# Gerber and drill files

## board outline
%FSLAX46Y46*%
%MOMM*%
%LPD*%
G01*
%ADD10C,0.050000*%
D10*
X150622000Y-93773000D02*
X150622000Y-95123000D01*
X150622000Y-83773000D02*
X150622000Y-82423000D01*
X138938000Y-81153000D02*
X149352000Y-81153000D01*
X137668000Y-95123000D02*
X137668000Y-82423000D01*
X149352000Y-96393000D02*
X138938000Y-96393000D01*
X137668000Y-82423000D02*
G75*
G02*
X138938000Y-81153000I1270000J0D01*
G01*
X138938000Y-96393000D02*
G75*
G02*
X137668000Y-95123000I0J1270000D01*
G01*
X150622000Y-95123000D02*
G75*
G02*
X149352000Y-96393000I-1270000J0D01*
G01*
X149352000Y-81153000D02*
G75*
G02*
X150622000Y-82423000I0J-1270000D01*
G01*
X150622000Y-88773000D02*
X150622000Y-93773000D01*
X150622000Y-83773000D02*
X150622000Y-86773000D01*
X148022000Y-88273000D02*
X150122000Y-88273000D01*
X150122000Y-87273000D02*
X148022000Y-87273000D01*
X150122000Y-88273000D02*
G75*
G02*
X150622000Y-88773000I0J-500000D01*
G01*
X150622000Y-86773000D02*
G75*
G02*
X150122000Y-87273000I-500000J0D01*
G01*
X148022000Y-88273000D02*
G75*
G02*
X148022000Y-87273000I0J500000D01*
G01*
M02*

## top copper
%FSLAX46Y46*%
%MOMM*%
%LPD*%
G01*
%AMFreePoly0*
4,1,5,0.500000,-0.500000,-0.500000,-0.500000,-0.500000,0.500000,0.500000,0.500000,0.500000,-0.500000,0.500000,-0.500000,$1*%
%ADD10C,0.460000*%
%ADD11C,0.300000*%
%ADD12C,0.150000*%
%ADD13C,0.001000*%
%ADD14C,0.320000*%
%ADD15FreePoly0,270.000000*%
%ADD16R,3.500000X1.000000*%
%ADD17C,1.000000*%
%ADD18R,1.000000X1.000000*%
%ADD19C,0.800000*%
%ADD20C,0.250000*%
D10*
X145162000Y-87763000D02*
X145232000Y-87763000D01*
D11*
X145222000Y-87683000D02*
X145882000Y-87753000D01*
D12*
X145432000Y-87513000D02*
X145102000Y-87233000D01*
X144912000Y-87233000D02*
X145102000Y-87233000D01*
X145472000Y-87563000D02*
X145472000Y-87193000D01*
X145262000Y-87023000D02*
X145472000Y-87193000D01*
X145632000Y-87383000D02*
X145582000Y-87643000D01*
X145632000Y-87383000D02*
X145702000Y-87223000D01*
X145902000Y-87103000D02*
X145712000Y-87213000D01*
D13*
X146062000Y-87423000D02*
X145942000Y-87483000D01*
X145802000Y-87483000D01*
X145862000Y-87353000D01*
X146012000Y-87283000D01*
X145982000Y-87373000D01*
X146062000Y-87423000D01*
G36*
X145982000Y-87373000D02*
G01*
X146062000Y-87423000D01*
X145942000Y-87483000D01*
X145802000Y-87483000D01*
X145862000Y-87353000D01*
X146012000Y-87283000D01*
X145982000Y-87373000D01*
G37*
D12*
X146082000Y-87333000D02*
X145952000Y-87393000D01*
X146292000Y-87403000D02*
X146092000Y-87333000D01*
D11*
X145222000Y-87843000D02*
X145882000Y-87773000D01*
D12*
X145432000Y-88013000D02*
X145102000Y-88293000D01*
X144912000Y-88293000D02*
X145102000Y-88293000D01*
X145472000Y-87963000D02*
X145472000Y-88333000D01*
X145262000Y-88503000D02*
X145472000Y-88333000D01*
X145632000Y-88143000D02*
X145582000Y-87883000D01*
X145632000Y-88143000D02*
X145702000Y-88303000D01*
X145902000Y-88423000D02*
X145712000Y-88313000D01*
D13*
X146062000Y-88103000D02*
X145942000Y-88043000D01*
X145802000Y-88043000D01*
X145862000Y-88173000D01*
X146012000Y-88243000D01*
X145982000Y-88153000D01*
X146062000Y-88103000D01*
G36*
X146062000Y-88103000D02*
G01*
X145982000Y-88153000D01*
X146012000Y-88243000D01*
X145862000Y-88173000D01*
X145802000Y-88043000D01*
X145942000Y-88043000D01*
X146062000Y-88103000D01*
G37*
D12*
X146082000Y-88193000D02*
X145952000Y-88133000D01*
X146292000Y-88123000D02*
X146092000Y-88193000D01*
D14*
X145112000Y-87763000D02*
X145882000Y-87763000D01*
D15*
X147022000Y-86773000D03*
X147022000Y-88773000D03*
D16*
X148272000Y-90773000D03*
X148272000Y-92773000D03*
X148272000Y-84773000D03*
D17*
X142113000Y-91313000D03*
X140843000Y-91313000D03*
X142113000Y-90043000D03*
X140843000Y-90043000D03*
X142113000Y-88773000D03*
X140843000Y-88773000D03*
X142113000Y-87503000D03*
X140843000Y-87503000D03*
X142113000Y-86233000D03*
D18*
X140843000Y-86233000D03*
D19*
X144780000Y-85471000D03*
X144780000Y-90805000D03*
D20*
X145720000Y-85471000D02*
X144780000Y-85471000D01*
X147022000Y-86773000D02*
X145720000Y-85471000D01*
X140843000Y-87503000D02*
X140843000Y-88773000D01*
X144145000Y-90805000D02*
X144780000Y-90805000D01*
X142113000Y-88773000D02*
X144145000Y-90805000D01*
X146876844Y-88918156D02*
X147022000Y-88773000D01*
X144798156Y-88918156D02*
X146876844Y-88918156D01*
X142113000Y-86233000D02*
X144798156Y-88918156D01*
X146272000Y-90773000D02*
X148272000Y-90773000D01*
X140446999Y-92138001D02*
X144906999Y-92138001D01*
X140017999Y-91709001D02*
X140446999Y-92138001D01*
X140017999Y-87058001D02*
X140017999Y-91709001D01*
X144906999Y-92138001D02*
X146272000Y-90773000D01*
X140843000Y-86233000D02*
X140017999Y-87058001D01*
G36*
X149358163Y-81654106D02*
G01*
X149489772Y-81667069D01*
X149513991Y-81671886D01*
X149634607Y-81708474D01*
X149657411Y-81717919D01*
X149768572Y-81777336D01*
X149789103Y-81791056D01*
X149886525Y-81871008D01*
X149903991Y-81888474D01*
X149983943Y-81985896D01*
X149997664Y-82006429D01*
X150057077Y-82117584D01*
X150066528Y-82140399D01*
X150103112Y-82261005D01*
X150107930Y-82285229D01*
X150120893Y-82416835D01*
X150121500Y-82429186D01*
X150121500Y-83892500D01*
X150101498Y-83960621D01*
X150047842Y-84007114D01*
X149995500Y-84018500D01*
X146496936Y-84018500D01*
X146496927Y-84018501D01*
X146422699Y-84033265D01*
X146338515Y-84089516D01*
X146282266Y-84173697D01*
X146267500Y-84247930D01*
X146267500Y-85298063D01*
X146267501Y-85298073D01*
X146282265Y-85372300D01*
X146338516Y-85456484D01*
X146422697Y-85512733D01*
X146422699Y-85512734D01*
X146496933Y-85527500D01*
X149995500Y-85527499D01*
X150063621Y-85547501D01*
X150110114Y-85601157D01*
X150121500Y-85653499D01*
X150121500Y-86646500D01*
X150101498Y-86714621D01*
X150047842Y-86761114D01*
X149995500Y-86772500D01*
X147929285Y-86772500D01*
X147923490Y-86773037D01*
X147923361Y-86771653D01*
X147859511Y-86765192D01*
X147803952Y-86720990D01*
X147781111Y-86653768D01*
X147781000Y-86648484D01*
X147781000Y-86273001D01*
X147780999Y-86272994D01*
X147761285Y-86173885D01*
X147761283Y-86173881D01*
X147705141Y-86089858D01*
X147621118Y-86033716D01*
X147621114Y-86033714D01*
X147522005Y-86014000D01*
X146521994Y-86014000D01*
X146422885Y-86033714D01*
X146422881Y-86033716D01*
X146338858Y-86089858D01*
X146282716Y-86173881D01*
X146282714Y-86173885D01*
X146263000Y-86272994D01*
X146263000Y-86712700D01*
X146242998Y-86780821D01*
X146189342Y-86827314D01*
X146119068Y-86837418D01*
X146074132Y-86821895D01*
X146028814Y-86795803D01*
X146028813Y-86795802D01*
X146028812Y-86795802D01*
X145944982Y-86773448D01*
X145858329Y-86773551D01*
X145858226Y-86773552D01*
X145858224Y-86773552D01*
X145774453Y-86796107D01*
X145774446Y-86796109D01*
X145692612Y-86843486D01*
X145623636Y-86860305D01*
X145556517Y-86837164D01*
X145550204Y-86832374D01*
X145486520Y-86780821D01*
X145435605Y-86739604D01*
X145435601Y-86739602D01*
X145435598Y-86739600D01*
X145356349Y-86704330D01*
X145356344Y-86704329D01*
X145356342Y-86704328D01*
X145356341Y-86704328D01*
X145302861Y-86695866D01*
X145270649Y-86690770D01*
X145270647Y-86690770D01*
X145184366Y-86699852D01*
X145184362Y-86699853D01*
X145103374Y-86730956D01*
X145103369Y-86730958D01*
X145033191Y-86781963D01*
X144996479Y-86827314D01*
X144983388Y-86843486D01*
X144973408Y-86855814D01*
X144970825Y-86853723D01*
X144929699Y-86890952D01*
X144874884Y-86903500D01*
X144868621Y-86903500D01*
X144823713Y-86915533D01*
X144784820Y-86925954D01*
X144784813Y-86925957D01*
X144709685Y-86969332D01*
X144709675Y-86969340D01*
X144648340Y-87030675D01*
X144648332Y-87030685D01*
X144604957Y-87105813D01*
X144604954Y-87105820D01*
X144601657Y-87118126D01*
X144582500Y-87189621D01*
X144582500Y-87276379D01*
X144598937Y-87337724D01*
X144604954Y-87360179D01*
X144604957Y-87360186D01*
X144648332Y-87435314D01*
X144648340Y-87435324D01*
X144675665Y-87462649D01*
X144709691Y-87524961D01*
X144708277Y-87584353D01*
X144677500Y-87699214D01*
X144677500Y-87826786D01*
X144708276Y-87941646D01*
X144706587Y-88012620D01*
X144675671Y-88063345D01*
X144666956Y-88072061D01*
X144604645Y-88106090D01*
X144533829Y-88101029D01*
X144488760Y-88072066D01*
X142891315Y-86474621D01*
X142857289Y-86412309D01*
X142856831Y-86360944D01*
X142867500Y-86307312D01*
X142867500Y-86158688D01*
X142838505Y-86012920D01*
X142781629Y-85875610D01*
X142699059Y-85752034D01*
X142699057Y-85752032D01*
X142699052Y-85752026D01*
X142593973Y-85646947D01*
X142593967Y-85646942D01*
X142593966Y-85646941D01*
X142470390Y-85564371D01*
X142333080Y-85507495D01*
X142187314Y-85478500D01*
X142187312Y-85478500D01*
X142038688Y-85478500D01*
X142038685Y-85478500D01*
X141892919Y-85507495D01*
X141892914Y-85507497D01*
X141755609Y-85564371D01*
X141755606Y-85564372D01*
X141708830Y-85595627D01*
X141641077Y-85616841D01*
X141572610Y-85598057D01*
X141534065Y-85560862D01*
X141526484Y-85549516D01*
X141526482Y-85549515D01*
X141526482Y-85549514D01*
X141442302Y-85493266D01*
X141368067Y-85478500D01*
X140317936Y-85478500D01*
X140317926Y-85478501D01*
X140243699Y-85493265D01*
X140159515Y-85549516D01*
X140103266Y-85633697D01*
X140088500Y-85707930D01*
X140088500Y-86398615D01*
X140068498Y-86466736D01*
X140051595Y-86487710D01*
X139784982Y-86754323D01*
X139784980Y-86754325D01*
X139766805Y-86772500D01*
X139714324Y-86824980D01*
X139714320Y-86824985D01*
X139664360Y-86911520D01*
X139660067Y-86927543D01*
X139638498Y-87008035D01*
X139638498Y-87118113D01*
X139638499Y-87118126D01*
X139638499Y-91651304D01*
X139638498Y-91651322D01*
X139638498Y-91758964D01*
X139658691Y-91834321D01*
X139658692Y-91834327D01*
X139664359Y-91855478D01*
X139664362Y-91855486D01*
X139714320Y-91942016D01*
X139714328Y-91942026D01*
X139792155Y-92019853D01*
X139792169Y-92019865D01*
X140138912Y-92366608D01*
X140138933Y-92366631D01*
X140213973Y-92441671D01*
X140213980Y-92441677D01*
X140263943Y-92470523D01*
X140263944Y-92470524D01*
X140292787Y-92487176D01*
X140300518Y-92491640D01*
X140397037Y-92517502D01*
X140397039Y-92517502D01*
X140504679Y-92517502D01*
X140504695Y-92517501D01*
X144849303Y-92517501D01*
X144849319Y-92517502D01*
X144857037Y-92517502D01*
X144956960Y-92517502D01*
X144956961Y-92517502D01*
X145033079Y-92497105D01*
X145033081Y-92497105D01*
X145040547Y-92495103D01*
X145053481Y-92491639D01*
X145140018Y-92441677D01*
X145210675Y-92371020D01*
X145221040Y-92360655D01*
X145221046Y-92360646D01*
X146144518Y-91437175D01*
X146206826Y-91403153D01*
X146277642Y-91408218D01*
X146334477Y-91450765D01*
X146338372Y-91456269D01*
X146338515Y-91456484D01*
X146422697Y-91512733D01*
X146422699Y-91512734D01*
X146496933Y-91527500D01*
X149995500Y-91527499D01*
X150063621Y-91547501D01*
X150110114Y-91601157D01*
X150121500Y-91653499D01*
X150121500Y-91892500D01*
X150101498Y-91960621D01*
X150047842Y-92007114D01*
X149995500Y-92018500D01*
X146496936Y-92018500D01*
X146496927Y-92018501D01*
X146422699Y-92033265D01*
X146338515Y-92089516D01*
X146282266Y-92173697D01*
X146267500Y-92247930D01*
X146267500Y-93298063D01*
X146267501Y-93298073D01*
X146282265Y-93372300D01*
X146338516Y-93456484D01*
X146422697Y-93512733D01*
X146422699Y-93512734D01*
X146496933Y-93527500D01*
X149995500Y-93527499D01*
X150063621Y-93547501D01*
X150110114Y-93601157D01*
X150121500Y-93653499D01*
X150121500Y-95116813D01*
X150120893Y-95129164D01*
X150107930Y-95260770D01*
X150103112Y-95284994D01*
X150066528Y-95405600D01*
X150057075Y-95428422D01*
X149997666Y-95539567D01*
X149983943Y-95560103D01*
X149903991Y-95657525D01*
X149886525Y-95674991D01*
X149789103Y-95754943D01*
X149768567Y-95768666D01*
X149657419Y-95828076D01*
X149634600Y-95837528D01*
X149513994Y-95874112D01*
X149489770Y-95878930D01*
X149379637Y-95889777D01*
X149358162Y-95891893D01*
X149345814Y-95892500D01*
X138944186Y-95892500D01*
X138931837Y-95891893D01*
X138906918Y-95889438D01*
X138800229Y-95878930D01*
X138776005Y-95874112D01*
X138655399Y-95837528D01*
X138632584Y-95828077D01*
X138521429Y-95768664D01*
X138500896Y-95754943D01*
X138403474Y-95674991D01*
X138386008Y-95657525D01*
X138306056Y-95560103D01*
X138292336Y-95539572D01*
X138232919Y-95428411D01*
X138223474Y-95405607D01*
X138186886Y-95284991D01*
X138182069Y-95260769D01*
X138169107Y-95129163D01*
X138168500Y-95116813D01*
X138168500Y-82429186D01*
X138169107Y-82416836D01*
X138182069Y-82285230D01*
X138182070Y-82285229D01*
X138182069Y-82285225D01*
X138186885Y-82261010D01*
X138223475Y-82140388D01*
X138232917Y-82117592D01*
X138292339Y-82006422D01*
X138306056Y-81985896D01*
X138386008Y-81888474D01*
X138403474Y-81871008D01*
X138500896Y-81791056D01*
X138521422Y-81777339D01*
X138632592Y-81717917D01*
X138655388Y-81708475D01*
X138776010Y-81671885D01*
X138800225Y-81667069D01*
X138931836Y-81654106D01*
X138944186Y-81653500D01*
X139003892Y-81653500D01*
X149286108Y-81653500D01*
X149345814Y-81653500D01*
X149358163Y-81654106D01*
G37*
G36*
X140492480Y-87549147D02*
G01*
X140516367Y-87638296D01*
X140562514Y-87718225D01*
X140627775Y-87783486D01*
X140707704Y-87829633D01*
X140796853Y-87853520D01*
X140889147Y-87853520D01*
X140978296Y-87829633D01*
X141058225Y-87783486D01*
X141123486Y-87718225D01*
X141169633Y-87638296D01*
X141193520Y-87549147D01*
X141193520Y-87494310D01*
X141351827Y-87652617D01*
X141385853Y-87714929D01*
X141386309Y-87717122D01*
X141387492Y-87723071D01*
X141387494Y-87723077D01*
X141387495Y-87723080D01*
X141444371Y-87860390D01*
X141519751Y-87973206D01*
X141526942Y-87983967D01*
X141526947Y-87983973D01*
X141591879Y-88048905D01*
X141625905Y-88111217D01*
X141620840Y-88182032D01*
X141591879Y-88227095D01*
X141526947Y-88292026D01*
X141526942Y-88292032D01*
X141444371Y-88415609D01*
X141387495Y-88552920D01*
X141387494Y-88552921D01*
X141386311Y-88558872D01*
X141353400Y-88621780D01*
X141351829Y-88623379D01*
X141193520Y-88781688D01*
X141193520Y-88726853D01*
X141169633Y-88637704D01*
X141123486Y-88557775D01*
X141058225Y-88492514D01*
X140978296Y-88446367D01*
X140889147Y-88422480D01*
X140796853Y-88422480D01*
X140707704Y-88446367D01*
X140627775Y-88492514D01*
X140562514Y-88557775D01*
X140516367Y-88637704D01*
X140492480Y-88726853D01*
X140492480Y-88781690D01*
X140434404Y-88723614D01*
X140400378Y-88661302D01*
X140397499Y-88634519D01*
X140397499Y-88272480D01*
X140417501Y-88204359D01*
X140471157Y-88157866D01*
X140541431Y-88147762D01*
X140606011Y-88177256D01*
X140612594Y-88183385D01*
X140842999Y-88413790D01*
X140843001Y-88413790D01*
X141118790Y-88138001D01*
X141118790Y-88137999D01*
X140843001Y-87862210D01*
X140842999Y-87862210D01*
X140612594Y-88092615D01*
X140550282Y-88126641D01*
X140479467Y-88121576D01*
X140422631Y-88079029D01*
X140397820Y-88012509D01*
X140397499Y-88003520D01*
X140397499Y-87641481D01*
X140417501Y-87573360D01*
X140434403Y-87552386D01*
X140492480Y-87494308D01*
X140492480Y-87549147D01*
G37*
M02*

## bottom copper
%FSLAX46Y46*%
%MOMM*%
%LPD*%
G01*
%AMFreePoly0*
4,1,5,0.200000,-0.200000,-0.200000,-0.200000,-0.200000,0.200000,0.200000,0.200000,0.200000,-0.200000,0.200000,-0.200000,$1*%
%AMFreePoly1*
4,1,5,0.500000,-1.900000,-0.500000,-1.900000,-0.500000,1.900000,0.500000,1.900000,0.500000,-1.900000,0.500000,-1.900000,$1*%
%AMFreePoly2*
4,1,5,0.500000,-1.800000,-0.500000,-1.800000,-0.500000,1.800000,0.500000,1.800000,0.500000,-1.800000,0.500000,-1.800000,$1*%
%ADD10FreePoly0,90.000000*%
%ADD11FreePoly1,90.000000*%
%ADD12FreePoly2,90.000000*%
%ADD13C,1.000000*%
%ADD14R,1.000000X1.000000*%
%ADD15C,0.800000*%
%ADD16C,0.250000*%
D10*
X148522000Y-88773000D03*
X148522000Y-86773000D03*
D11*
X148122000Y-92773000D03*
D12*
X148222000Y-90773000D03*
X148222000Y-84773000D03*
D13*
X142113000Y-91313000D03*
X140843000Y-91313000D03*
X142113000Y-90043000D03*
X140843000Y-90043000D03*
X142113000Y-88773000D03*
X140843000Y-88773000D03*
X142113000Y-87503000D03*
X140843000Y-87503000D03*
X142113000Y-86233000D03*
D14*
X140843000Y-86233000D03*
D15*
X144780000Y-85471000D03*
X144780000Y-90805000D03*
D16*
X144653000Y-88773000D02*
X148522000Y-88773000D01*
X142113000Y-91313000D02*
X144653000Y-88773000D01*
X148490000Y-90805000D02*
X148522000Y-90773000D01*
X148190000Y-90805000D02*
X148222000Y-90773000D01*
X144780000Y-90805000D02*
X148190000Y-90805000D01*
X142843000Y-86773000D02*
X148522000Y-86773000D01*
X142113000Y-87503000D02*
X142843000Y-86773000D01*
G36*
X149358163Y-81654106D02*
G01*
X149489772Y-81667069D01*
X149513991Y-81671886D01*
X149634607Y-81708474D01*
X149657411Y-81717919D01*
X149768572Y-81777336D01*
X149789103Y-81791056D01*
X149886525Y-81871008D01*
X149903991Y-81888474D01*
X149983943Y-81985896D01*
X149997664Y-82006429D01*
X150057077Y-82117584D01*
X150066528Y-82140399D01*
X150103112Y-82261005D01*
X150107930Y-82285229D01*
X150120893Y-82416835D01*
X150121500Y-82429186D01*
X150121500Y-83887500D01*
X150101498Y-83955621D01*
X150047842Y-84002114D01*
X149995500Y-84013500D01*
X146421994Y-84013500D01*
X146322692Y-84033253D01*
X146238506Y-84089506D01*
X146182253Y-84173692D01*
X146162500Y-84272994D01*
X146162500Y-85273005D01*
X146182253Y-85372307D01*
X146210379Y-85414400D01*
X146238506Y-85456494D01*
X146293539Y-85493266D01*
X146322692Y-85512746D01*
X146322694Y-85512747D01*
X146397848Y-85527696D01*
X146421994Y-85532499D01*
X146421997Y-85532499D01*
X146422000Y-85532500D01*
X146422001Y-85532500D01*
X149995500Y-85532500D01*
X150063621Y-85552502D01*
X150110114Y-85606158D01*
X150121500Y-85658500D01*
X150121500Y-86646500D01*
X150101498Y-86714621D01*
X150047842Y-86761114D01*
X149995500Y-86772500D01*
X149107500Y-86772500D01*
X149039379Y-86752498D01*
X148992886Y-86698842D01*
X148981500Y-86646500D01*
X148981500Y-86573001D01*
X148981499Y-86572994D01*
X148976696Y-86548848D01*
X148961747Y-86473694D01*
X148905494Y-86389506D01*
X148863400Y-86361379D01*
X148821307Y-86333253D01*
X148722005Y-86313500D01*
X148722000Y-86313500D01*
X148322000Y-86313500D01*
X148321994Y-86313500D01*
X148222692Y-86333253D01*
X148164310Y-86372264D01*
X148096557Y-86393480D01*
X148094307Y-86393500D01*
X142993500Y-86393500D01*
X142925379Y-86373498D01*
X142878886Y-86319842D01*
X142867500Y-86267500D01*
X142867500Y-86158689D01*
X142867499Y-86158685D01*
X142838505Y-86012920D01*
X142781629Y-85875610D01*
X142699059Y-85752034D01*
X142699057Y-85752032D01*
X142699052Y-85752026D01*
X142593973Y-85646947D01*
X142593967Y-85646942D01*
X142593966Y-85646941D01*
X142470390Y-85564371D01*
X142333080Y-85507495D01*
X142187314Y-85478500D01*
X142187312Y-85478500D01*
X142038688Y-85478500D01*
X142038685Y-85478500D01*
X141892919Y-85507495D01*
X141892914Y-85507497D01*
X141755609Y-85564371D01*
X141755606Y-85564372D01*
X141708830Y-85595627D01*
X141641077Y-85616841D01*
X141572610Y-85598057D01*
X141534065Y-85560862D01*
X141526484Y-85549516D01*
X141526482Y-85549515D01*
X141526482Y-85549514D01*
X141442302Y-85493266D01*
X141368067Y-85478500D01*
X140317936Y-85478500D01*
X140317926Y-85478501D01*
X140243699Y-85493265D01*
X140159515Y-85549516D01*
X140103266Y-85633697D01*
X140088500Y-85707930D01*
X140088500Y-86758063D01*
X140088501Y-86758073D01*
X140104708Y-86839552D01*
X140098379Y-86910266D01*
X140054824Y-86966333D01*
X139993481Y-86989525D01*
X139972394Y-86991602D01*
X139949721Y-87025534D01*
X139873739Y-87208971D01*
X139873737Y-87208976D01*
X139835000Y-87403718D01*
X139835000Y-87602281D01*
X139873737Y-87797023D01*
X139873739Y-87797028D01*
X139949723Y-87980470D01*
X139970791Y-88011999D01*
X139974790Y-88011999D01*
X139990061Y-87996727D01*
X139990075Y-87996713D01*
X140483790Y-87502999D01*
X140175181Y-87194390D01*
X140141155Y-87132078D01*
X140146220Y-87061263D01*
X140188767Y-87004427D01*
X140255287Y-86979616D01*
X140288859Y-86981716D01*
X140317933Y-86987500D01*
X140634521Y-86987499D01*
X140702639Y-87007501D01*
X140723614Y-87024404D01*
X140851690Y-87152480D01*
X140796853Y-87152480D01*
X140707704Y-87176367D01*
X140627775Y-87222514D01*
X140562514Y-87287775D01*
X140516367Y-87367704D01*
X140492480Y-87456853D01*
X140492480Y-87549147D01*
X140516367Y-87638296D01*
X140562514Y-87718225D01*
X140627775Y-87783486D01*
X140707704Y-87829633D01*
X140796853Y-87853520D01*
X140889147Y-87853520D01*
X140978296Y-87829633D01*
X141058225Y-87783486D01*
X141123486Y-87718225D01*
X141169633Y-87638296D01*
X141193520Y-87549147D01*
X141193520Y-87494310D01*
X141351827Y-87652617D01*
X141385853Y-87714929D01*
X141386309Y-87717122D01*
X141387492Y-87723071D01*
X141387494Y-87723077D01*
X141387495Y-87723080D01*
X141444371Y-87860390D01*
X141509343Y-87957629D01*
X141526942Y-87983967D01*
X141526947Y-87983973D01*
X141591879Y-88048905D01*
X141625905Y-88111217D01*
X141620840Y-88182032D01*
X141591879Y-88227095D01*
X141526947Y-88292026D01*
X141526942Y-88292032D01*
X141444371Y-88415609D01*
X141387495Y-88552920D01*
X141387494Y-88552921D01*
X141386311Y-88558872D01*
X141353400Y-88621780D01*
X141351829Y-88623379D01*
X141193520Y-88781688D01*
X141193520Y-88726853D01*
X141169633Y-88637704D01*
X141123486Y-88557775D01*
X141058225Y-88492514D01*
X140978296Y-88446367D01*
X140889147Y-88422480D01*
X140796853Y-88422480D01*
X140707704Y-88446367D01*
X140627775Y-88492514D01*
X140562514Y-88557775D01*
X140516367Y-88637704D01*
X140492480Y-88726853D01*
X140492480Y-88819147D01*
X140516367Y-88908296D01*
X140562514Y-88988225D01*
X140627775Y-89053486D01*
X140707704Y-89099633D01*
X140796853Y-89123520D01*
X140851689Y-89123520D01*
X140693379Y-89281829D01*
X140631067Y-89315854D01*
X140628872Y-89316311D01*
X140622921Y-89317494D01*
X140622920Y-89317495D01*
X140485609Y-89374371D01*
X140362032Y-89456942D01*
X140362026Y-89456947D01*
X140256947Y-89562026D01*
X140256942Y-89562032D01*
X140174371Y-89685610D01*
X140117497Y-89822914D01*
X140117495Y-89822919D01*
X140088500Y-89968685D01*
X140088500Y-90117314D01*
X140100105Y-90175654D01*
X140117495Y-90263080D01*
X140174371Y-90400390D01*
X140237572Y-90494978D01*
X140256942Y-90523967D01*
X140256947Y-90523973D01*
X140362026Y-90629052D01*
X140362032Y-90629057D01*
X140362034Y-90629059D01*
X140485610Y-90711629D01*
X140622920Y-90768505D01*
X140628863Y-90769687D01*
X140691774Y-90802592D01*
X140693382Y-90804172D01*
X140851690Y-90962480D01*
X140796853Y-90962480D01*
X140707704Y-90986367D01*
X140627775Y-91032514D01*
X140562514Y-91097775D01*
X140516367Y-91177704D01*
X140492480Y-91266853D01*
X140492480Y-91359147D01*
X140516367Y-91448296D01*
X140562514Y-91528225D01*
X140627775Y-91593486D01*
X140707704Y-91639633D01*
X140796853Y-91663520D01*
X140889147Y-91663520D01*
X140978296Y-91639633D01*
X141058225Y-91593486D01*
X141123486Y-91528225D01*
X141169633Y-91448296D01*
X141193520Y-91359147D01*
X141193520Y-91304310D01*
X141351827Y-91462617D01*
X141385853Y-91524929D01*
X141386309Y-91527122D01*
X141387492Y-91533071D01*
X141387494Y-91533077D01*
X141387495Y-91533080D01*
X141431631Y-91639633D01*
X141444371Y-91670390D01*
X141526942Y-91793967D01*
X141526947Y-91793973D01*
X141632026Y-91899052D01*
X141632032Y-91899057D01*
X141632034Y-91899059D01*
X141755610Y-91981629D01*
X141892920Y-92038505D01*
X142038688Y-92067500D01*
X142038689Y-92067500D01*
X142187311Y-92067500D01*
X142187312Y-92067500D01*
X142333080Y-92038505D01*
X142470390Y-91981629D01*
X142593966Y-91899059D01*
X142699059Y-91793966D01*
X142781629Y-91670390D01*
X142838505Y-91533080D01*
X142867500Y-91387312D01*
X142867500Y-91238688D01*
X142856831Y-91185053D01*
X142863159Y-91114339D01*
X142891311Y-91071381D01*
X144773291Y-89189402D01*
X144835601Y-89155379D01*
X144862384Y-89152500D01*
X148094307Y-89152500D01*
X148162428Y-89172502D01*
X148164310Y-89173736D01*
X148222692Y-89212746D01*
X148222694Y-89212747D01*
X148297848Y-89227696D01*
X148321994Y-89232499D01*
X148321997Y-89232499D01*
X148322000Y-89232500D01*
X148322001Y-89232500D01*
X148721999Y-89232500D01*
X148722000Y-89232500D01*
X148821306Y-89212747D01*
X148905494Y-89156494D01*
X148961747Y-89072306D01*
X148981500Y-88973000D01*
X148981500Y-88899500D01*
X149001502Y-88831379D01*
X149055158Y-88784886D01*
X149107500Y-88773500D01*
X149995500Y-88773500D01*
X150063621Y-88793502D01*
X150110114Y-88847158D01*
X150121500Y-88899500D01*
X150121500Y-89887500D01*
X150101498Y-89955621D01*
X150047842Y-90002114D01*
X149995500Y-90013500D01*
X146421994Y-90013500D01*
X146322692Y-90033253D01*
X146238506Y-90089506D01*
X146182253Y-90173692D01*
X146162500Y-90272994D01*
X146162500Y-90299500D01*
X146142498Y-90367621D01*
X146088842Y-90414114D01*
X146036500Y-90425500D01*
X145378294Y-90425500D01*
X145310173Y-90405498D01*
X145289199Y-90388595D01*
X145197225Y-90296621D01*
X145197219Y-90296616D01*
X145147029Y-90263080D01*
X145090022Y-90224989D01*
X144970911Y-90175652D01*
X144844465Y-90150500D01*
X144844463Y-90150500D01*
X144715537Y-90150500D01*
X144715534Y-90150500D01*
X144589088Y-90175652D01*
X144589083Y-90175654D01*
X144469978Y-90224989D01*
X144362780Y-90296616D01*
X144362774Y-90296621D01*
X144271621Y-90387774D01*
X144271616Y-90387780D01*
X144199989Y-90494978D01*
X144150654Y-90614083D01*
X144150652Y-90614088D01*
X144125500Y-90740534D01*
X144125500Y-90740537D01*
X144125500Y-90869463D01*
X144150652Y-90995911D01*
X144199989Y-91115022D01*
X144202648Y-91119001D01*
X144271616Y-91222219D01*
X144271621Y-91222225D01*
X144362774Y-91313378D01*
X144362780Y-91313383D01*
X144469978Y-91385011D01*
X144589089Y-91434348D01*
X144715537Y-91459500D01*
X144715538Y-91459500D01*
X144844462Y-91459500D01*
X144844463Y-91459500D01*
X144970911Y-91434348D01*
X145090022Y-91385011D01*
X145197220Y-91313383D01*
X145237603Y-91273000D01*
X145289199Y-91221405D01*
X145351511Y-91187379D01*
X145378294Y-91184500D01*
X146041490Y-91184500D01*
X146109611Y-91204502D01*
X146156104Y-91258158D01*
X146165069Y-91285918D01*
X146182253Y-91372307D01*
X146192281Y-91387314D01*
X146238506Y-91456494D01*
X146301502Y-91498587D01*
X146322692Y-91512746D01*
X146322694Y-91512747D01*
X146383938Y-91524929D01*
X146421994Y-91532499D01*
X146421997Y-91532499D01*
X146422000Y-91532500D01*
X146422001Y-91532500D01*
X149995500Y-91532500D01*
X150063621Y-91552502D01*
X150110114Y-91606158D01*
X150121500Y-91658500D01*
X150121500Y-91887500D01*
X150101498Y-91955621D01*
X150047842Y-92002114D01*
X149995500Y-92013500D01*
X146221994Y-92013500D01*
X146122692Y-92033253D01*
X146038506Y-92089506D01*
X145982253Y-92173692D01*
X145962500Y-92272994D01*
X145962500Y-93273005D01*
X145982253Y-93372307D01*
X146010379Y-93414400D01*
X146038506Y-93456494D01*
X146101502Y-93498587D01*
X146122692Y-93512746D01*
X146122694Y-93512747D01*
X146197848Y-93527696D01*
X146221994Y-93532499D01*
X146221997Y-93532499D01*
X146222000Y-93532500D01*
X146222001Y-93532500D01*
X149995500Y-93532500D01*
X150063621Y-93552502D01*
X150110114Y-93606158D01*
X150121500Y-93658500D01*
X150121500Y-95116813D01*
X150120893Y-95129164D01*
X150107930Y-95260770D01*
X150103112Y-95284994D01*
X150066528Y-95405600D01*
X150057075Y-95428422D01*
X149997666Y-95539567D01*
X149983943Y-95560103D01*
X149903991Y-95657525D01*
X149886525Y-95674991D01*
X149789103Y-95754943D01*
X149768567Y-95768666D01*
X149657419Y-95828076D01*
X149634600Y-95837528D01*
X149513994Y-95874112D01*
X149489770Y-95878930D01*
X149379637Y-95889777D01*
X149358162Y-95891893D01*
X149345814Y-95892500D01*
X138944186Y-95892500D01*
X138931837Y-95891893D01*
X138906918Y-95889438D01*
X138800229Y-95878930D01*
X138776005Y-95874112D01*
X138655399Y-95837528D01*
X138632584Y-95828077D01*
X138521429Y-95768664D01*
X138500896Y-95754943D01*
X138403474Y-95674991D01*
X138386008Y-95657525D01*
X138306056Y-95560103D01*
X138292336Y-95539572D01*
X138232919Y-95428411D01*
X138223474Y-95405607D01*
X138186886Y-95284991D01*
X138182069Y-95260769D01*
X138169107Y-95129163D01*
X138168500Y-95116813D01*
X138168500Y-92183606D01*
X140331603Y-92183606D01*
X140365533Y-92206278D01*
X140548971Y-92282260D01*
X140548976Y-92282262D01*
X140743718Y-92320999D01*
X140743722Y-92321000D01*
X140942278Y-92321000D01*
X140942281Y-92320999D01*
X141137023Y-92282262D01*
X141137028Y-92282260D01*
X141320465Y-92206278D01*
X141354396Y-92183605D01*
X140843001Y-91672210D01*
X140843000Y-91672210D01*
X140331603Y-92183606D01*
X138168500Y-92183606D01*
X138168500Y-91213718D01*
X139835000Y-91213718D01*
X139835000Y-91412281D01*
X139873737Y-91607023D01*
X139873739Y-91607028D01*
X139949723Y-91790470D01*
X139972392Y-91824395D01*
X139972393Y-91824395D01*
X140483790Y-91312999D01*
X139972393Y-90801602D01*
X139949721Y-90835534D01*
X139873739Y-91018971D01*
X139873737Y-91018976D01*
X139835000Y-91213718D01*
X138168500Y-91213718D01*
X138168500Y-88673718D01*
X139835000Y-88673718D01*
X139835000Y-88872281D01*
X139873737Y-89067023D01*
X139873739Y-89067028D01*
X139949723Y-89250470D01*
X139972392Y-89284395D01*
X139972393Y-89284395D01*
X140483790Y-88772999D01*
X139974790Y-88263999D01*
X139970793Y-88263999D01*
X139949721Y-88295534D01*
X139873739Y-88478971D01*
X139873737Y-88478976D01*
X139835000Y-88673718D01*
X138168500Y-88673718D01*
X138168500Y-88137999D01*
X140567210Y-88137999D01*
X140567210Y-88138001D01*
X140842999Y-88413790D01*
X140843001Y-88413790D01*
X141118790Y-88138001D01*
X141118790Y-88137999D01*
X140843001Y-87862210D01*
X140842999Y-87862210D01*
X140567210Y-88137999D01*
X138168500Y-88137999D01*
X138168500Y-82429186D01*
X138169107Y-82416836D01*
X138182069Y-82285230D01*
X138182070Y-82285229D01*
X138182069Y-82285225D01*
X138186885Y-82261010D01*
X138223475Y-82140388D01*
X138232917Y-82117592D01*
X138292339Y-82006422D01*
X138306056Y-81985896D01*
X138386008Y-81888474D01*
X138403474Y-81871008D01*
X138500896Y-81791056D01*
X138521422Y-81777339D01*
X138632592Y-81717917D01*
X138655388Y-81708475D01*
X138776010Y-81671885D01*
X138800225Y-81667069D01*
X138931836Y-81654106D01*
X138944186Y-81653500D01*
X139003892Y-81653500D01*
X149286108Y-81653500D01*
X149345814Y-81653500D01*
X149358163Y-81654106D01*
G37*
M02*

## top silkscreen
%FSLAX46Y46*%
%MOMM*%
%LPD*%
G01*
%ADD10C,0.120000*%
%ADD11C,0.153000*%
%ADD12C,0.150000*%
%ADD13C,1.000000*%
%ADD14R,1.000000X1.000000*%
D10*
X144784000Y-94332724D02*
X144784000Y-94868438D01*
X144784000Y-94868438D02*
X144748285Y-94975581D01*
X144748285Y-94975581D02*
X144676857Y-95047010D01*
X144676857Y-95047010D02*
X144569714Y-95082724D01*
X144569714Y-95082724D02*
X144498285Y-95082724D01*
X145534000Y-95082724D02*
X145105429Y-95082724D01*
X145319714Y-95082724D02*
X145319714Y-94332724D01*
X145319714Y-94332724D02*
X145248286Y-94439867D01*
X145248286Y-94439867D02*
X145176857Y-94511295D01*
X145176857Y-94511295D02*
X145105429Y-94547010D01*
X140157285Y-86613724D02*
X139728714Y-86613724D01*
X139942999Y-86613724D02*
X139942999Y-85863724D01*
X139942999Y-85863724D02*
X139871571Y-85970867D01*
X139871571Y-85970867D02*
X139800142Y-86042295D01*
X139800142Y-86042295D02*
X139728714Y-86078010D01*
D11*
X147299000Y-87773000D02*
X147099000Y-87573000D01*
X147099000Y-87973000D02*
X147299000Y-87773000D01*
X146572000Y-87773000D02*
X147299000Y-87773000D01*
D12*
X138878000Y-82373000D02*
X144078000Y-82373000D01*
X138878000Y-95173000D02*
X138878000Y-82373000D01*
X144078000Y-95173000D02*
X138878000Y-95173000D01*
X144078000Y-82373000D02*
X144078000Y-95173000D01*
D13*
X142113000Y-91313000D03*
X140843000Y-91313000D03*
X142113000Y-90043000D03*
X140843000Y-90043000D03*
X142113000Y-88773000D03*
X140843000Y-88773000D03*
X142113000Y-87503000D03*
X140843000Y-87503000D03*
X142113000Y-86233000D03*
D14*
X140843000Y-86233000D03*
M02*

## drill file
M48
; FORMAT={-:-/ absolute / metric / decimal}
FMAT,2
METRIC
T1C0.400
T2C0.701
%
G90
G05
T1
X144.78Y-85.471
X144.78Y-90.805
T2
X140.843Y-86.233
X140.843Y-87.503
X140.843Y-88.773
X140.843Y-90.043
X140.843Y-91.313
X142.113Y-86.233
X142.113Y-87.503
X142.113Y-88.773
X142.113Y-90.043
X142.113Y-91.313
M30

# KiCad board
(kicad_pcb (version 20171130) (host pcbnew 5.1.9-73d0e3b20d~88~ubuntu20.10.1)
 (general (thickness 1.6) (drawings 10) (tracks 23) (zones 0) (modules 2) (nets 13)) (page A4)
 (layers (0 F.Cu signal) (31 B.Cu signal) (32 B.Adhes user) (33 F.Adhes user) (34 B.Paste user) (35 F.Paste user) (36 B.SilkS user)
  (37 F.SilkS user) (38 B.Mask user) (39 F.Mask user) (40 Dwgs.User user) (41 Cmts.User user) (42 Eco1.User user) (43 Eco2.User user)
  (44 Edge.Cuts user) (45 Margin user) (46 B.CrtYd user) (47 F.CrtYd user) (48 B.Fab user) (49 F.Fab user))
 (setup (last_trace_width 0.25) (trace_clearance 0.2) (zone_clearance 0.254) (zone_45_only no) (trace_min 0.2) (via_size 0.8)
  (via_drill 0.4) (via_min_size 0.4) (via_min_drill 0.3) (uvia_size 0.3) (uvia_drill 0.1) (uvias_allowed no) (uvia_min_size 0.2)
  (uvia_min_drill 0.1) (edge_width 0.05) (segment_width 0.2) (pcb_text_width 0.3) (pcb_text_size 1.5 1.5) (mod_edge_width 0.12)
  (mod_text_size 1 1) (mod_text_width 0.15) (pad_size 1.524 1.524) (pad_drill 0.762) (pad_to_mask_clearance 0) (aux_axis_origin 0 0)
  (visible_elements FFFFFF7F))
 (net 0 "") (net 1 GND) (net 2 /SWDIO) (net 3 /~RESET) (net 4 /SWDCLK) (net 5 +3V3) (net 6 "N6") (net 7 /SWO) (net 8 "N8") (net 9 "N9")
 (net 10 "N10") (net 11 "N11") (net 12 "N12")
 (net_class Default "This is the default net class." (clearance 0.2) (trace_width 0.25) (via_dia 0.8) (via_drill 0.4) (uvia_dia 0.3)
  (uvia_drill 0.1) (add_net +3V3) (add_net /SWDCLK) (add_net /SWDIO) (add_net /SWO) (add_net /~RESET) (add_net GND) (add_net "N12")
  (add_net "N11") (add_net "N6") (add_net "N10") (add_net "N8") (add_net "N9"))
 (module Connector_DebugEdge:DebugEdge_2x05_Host (layer F.Cu) (at 150.622 88.773 270)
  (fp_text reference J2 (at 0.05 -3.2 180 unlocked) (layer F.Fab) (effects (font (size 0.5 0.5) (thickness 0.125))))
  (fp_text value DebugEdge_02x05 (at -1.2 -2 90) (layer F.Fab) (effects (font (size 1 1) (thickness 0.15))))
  (fp_line (start -1.01 5.46) (end -1.01 5.39) (layer F.Cu) (width 0.46))
  (fp_line (start -1.09 5.4) (end -1.02 4.74) (layer F.Cu) (width 0.3))
  (fp_line (start -1.26 5.19) (end -1.54 5.52) (layer F.Cu) (width 0.15))
  (fp_line (start -1.54 5.71) (end -1.54 5.52) (layer F.Cu) (width 0.15))
  (fp_line (start -1.21 5.15) (end -1.58 5.15) (layer F.Cu) (width 0.15))
  (fp_line (start -1.75 5.36) (end -1.58 5.15) (layer F.Cu) (width 0.15))
  (fp_line (start -1.39 4.99) (end -1.13 5.04) (layer F.Cu) (width 0.15))
  (fp_line (start -1.39 4.99) (end -1.55 4.92) (layer F.Cu) (width 0.15))
  (fp_line (start -1.67 4.72) (end -1.56 4.91) (layer F.Cu) (width 0.15))
  (fp_poly (pts (xy -1.35 4.56) (xy -1.29 4.68) (xy -1.29 4.82) (xy -1.42 4.76) (xy -1.49 4.61) (xy -1.4 4.64)) (layer F.Cu) (width 0.001))
  (fp_line (start -1.44 4.54) (end -1.38 4.67) (layer F.Cu) (width 0.15))
  (fp_line (start -1.37 4.33) (end -1.44 4.53) (layer F.Cu) (width 0.15))
  (fp_line (start 0 0) (end 5 0) (layer Edge.Cuts) (width 0.05))
  (fp_line (start -5 0) (end -2 0) (layer Edge.Cuts) (width 0.05))
  (fp_line (start -0.5 2.6) (end -0.5 0.5) (layer Edge.Cuts) (width 0.05))
  (fp_line (start -1.5 0.5) (end -1.5 2.6) (layer Edge.Cuts) (width 0.05))
  (fp_line (start -1 3.323) (end -1.2 3.523) (layer F.SilkS) (width 0.153))
  (fp_line (start -0.8 3.523) (end -1 3.323) (layer F.SilkS) (width 0.153))
  (fp_line (start -1 4.05) (end -1 3.323) (layer F.SilkS) (width 0.153))
  (fp_line (start -0.93 5.4) (end -1 4.74) (layer F.Cu) (width 0.3))
  (fp_line (start -0.76 5.19) (end -0.48 5.52) (layer F.Cu) (width 0.15))
  (fp_line (start -0.48 5.71) (end -0.48 5.52) (layer F.Cu) (width 0.15))
  (fp_line (start -0.81 5.15) (end -0.44 5.15) (layer F.Cu) (width 0.15))
  (fp_line (start -0.27 5.36) (end -0.44 5.15) (layer F.Cu) (width 0.15))
  (fp_line (start -0.63 4.99) (end -0.89 5.04) (layer F.Cu) (width 0.15))
  (fp_line (start -0.63 4.99) (end -0.47 4.92) (layer F.Cu) (width 0.15))
  (fp_line (start -0.35 4.72) (end -0.46 4.91) (layer F.Cu) (width 0.15))
  (fp_poly (pts (xy -0.67 4.56) (xy -0.73 4.68) (xy -0.73 4.82) (xy -0.6 4.76) (xy -0.53 4.61) (xy -0.62 4.64)) (layer F.Cu) (width 0.001))
  (fp_line (start -0.58 4.54) (end -0.64 4.67) (layer F.Cu) (width 0.15))
  (fp_line (start -0.65 4.33) (end -0.58 4.53) (layer F.Cu) (width 0.15))
  (fp_line (start -1.01 5.51) (end -1.01 4.74) (layer F.Cu) (width 0.32))
  (fp_arc (start 0 0.5) (end 0 0) (angle -90) (layer Edge.Cuts) (width 0.05))
  (fp_arc (start -2 0.5) (end -1.5 0.5) (angle -90) (layer Edge.Cuts) (width 0.05))
  (fp_arc (start -1 2.6) (end -1.5 2.6) (angle -180) (layer Edge.Cuts) (width 0.05))
  (pad 1 smd custom (at -2 3.6 270) (size 1 1) (layers F.Cu F.Mask) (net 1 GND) (zone_connect 0) (options (clearance outline) (anchor rect))
   (primitives))
  (pad 2 smd custom (at 0 3.6 270) (size 1 1) (layers F.Cu F.Mask) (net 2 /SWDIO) (zone_connect 0)
   (options (clearance outline) (anchor rect)) (primitives))
  (pad 4 smd custom (at 0 2.1 90) (size 0.4 0.4) (layers B.Cu B.Mask) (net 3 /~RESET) (zone_connect 0)
   (options (clearance outline) (anchor rect)) (primitives))
  (pad 3 smd custom (at -2 2.1 90) (size 0.4 0.4) (layers B.Cu B.Mask) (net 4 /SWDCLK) (zone_connect 0)
   (options (clearance outline) (anchor rect)) (primitives))
  (pad 5 smd rect (at 2 2.35 270) (size 1 3.5) (layers F.Cu F.Mask) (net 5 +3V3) (zone_connect 0))
  (pad 10 smd custom (at 4 2.5 90) (size 1 3.8) (layers B.Cu B.Mask) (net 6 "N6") (zone_connect 0)
   (options (clearance outline) (anchor rect)) (primitives))
  (pad 6 smd custom (at 2 2.4 90) (size 1 3.6) (layers B.Cu B.Mask) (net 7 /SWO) (zone_connect 0)
   (options (clearance outline) (anchor rect)) (primitives))
  (pad 8 smd custom (at -4 2.4 90) (size 1 3.6) (layers B.Cu B.Mask) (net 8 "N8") (zone_connect 0)
   (options (clearance outline) (anchor rect)) (primitives))
  (pad 9 smd rect (at 4 2.35 270) (size 1 3.5) (layers F.Cu F.Mask) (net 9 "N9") (zone_connect 0))
  (pad 7 smd rect (at -4 2.35 270) (size 1 3.5) (layers F.Cu F.Mask) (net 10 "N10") (zone_connect 0)))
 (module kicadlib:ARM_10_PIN (layer F.Cu) (at 141.478 88.773)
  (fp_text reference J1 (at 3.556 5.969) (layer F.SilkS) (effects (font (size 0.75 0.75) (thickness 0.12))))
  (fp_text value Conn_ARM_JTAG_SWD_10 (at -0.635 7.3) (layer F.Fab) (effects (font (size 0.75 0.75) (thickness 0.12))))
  (fp_line (start -2.6 -6.4) (end 2.6 -6.4) (layer F.SilkS) (width 0.15))
  (fp_line (start -2.6 6.4) (end -2.6 -6.4) (layer F.SilkS) (width 0.15))
  (fp_line (start 2.6 6.4) (end -2.6 6.4) (layer F.SilkS) (width 0.15))
  (fp_line (start 2.6 -6.4) (end 2.6 6.4) (layer F.SilkS) (width 0.15))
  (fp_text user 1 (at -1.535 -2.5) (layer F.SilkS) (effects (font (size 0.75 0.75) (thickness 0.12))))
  (pad 10 thru_hole circle (at 0.635 2.54) (size 1 1) (drill 0.70104) (layers *.Cu *.Mask F.SilkS) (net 3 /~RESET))
  (pad 9 thru_hole circle (at -0.635 2.54) (size 1 1) (drill 0.70104) (layers *.Cu *.Mask F.SilkS) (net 1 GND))
  (pad 8 thru_hole circle (at 0.635 1.27) (size 1 1) (drill 0.70104) (layers *.Cu *.Mask F.SilkS) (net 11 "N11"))
  (pad 7 thru_hole circle (at -0.635 1.27) (size 1 1) (drill 0.70104) (layers *.Cu *.Mask F.SilkS) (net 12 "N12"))
  (pad 6 thru_hole circle (at 0.635 0) (size 1 1) (drill 0.70104) (layers *.Cu *.Mask F.SilkS) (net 7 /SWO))
  (pad 5 thru_hole circle (at -0.635 0) (size 1 1) (drill 0.70104) (layers *.Cu *.Mask F.SilkS) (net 1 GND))
  (pad 4 thru_hole circle (at 0.635 -1.27) (size 1 1) (drill 0.70104) (layers *.Cu *.Mask F.SilkS) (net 4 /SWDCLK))
  (pad 3 thru_hole circle (at -0.635 -1.27) (size 1 1) (drill 0.70104) (layers *.Cu *.Mask F.SilkS) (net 1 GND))
  (pad 2 thru_hole circle (at 0.635 -2.54) (size 1 1) (drill 0.70104) (layers *.Cu *.Mask F.SilkS) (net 2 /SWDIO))
  (pad 1 thru_hole rect (at -0.635 -2.54) (size 1 1) (drill 0.70104) (layers *.Cu *.Mask F.SilkS) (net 5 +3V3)))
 (gr_line (start 150.622 93.773) (end 150.622 95.123) (layer Edge.Cuts) (width 0.05))
 (gr_line (start 150.622 83.773) (end 150.622 82.423) (layer Edge.Cuts) (width 0.05))
 (gr_line (start 138.938 81.153) (end 149.352 81.153) (layer Edge.Cuts) (width 0.05))
 (gr_line (start 137.668 95.123) (end 137.668 82.423) (layer Edge.Cuts) (width 0.05))
 (gr_line (start 149.352 96.393) (end 138.938 96.393) (layer Edge.Cuts) (width 0.05))
 (gr_arc (start 138.938 82.423) (end 138.938 81.153) (angle -90) (layer Edge.Cuts) (width 0.05))
 (gr_arc (start 138.938 95.123) (end 137.668 95.123) (angle -90) (layer Edge.Cuts) (width 0.05))
 (gr_arc (start 149.352 95.123) (end 149.352 96.393) (angle -90) (layer Edge.Cuts) (width 0.05))
 (gr_arc (start 149.352 82.423) (end 150.622 82.423) (angle -90) (layer Edge.Cuts) (width 0.05))
 (segment (start 144.653 88.773) (end 148.522 88.773) (width 0.25) (layer B.Cu) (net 3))
 (segment (start 142.113 91.313) (end 144.653 88.773) (width 0.25) (layer B.Cu) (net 3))
 (via (at 144.78 85.471) (size 0.8) (drill 0.4) (layers F.Cu B.Cu) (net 1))
 (segment (start 145.72 85.471) (end 144.78 85.471) (width 0.25) (layer F.Cu) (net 1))
 (segment (start 147.022 86.773) (end 145.72 85.471) (width 0.25) (layer F.Cu) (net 1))
 (segment (start 140.843 87.503) (end 140.843 88.773) (width 0.25) (layer F.Cu) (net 1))
 (segment (start 148.49 90.805) (end 148.522 90.773) (width 0.25) (layer B.Cu) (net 7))
 (via (at 144.78 90.805) (size 0.8) (drill 0.4) (layers F.Cu B.Cu) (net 7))
 (segment (start 144.145 90.805) (end 144.78 90.805) (width 0.25) (layer F.Cu) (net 7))
 (segment (start 142.113 88.773) (end 144.145 90.805) (width 0.25) (layer F.Cu) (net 7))
 (segment (start 148.19 90.805) (end 148.222 90.773) (width 0.25) (layer B.Cu) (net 7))
 (segment (start 144.78 90.805) (end 148.19 90.805) (width 0.25) (layer B.Cu) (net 7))
 (segment (start 142.843 86.773) (end 148.522 86.773) (width 0.25) (layer B.Cu) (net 4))
 (segment (start 142.113 87.503) (end 142.843 86.773) (width 0.25) (layer B.Cu) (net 4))
 (segment (start 146.876844 88.918156) (end 147.022 88.773) (width 0.25) (layer F.Cu) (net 2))
 (segment (start 144.798156 88.918156) (end 146.876844 88.918156) (width 0.25) (layer F.Cu) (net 2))
 (segment (start 142.113 86.233) (end 144.798156 88.918156) (width 0.25) (layer F.Cu) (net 2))
 (segment (start 146.272 90.773) (end 148.272 90.773) (width 0.25) (layer F.Cu) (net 5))
 (segment (start 140.446999 92.138001) (end 144.906999 92.138001) (width 0.25) (layer F.Cu) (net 5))
 (segment (start 140.017999 91.709001) (end 140.446999 92.138001) (width 0.25) (layer F.Cu) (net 5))
 (segment (start 140.017999 87.058001) (end 140.017999 91.709001) (width 0.25) (layer F.Cu) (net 5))
 (segment (start 144.906999 92.138001) (end 146.272 90.773) (width 0.25) (layer F.Cu) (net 5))
 (segment (start 140.843 86.233) (end 140.017999 87.058001) (width 0.25) (layer F.Cu) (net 5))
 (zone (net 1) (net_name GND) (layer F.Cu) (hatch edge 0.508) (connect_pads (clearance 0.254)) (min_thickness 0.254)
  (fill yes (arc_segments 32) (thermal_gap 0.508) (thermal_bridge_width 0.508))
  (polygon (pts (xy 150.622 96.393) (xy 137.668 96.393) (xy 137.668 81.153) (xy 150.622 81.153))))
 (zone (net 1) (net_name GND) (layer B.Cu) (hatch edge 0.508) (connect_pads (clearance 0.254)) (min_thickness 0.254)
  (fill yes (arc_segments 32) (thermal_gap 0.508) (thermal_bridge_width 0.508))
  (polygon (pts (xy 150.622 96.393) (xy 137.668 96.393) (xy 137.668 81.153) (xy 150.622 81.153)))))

